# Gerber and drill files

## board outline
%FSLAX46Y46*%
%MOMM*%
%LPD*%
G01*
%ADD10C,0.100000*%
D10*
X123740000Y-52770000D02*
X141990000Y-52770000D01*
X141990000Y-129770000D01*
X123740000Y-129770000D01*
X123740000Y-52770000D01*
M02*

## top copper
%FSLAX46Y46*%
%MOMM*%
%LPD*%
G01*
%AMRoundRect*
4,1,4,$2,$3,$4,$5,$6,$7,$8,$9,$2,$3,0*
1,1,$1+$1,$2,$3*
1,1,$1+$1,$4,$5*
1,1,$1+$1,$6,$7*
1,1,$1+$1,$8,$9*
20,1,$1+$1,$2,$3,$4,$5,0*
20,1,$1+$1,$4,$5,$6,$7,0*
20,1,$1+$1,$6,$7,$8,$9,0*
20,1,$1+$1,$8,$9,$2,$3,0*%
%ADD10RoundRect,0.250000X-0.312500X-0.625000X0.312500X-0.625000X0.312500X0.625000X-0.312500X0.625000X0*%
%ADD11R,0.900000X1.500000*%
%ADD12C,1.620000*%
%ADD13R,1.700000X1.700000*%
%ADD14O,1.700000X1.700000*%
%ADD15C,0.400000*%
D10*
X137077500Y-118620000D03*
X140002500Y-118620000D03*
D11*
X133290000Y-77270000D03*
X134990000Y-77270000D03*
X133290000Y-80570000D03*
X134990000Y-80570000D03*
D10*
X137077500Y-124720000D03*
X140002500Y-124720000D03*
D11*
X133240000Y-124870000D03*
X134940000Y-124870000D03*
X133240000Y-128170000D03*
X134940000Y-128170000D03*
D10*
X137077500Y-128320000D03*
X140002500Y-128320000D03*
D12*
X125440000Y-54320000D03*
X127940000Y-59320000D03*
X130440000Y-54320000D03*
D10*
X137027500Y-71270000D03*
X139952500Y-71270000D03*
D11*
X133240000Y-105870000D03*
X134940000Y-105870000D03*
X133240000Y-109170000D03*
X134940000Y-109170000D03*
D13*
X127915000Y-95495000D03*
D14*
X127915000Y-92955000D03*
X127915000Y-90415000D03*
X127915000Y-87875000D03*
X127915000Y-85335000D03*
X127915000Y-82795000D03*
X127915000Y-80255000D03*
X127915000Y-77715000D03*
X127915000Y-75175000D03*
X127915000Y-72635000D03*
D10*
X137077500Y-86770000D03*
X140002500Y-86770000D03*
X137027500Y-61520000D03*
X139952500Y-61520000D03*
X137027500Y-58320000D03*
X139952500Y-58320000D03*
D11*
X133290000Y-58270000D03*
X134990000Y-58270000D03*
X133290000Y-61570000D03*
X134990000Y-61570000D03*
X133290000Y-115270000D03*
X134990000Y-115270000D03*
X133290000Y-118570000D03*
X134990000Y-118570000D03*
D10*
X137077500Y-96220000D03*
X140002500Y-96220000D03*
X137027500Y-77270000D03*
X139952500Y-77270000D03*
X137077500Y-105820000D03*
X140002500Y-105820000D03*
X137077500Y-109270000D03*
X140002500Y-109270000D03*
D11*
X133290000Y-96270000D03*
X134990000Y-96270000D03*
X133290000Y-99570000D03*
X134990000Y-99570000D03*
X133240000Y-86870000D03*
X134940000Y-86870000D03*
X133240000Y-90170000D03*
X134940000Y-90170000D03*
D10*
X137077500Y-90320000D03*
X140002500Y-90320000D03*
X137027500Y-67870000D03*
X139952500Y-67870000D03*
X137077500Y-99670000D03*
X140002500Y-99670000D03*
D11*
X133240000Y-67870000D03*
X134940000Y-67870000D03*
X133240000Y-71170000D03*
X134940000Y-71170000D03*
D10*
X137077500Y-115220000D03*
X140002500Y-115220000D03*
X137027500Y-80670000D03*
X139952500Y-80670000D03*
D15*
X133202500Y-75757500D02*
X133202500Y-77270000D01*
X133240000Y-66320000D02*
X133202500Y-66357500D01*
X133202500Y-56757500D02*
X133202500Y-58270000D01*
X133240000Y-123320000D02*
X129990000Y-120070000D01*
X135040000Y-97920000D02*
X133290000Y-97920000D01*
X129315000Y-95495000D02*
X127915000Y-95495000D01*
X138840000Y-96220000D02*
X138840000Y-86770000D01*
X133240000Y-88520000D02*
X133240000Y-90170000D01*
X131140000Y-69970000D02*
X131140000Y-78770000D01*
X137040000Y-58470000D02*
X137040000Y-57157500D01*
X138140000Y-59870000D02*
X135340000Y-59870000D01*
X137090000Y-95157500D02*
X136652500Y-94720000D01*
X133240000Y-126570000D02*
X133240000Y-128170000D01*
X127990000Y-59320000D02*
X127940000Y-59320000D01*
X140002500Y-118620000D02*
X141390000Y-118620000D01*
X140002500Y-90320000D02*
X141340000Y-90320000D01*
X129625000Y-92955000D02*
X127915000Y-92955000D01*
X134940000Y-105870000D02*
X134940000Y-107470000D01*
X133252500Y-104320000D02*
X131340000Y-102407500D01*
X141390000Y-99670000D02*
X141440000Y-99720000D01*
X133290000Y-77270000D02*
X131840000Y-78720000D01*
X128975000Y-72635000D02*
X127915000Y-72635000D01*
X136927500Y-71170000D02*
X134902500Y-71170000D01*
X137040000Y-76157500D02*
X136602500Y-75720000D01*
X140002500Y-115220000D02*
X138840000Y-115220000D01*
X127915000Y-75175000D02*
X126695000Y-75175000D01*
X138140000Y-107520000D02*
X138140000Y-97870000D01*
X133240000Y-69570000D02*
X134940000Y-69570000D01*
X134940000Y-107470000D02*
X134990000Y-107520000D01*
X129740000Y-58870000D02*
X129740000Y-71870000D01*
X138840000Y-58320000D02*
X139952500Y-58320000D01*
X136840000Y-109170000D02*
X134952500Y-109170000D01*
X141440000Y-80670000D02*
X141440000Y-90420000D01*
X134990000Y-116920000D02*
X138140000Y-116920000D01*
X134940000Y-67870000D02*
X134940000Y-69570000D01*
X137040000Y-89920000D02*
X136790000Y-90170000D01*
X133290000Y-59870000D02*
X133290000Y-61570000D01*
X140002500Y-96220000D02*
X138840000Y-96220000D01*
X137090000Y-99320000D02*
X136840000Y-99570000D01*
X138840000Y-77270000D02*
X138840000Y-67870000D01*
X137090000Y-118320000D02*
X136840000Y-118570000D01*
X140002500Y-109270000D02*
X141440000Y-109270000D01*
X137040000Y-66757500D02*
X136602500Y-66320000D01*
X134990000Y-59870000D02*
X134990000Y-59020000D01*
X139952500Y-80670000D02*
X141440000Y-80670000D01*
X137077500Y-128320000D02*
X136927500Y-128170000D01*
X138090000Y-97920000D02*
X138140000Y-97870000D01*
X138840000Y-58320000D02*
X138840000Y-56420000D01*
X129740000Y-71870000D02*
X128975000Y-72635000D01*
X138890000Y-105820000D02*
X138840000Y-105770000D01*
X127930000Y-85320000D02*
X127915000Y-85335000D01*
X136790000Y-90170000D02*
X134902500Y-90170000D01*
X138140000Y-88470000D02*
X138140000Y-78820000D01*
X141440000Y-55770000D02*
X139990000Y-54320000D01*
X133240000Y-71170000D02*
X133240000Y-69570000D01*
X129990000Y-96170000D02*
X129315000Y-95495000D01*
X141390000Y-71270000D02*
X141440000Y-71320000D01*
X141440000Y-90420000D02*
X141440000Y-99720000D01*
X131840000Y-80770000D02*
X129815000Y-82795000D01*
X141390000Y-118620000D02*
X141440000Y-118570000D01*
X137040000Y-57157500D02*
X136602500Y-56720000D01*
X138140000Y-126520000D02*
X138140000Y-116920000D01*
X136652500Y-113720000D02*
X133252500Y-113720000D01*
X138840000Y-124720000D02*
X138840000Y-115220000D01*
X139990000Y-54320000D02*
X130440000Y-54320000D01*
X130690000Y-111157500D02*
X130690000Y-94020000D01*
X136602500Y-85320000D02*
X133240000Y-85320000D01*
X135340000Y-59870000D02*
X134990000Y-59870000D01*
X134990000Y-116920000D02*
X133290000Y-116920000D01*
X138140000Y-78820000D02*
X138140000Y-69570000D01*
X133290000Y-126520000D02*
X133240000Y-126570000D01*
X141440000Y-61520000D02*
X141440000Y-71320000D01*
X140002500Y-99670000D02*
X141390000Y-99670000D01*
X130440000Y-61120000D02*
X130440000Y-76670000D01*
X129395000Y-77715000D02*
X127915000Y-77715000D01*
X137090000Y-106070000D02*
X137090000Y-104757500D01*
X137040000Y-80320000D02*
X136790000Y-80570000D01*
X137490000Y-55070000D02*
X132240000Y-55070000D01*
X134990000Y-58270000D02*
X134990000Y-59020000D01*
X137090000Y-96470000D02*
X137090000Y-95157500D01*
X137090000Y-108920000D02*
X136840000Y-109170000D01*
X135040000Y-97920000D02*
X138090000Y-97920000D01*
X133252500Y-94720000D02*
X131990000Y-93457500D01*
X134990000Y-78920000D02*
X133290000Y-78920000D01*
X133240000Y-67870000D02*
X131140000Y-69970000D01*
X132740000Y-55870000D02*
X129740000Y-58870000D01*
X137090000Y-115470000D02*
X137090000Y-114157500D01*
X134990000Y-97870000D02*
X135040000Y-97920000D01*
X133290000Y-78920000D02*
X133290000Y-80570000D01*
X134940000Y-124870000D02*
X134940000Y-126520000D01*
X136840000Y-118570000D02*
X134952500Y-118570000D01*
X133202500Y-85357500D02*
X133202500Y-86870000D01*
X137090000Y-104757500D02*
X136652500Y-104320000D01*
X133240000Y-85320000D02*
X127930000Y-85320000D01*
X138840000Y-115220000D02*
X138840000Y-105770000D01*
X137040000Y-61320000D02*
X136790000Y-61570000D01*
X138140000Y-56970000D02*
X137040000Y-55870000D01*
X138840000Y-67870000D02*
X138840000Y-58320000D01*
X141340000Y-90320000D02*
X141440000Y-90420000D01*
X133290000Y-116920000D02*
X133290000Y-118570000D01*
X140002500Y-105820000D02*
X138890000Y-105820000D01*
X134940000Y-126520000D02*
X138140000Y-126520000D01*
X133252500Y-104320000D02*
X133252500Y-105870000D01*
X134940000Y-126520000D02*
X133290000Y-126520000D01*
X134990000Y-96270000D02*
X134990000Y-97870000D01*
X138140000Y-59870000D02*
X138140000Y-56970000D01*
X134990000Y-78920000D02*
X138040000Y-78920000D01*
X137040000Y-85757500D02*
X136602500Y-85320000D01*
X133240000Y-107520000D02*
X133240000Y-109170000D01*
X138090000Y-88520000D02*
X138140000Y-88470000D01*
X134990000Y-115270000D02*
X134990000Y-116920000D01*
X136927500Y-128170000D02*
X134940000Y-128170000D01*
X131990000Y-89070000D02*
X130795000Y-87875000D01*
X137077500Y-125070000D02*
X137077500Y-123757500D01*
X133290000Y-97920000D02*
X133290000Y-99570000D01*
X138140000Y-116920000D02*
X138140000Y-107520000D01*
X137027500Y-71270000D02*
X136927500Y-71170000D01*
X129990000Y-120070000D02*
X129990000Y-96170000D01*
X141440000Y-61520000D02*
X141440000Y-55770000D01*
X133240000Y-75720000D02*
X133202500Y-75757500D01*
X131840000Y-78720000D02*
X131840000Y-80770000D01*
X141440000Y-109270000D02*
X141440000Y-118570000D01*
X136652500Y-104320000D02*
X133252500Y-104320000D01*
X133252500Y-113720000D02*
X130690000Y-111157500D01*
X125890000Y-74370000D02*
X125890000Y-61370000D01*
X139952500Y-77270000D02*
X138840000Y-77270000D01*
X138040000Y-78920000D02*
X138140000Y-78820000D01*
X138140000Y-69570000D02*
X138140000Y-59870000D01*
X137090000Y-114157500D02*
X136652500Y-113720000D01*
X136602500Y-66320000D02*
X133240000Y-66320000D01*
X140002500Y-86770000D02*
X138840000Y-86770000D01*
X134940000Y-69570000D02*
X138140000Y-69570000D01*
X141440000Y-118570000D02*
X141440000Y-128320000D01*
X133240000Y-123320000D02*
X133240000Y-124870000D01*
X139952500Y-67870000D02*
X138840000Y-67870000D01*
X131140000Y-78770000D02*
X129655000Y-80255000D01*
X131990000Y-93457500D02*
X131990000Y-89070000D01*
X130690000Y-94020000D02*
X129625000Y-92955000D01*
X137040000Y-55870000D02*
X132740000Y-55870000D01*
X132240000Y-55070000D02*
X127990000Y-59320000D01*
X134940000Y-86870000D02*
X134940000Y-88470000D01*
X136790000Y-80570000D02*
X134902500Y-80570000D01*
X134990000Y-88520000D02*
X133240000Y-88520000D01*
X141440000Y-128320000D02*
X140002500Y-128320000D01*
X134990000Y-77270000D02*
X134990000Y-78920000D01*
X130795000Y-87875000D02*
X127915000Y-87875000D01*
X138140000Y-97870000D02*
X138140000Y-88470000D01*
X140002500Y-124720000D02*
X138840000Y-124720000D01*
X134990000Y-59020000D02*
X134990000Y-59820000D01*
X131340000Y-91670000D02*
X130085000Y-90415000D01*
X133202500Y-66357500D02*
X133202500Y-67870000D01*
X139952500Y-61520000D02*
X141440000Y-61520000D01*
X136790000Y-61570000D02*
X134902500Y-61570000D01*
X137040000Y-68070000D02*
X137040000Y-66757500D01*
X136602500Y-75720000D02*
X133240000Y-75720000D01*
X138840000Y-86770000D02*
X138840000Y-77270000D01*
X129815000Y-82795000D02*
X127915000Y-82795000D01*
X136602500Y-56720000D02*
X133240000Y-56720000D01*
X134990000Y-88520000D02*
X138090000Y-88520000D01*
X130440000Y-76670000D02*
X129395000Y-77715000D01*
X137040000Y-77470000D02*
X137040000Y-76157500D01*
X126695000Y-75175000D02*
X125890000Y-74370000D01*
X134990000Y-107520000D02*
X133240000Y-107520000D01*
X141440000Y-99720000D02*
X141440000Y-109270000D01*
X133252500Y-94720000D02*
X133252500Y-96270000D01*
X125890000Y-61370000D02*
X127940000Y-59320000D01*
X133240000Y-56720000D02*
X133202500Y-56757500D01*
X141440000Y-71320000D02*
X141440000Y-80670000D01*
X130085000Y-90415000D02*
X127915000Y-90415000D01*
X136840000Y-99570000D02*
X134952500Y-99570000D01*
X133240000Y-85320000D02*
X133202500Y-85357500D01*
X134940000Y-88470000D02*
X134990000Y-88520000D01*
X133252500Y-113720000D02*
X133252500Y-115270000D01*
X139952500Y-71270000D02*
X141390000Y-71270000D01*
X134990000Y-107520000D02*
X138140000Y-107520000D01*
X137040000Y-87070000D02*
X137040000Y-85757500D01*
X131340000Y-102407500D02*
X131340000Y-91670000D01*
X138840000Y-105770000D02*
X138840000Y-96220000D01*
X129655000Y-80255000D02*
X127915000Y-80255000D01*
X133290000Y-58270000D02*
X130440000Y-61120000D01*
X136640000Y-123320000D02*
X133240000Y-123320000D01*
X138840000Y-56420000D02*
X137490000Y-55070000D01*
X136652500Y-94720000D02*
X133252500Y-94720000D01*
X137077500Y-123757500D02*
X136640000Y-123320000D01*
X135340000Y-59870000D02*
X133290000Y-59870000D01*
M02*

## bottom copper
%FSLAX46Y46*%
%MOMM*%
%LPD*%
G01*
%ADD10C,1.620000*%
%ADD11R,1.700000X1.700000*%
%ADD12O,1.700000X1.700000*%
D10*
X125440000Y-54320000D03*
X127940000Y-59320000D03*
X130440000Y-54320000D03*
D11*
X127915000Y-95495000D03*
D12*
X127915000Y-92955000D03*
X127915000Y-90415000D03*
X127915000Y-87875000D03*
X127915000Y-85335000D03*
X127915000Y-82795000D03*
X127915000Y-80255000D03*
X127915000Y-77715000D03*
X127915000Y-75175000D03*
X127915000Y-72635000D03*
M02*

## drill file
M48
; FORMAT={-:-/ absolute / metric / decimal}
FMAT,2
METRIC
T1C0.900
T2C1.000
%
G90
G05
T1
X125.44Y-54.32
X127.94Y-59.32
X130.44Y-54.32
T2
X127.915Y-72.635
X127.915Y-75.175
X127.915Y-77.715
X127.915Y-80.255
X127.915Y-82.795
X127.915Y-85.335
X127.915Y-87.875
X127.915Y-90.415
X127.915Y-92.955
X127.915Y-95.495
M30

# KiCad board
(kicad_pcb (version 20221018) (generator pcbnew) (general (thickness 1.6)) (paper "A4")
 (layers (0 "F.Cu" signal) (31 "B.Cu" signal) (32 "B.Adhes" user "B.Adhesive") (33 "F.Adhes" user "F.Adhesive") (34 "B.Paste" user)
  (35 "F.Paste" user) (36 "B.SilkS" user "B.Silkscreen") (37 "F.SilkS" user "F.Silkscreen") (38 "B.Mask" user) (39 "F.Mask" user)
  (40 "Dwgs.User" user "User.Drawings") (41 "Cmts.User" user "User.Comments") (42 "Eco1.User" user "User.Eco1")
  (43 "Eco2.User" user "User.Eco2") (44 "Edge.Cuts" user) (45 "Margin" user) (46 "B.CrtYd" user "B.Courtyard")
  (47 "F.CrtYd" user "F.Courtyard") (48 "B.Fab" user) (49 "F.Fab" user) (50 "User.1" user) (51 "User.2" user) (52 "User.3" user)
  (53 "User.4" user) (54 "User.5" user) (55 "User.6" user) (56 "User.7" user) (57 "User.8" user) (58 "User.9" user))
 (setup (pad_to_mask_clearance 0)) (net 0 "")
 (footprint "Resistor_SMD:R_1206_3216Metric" (layer "F.Cu") (at 138.54 118.62)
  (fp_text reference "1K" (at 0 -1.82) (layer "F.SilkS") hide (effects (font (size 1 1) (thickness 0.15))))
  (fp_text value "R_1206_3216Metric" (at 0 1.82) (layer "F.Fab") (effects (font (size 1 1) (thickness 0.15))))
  (pad "1" smd roundrect (at -1.4625 0) (size 1.125 1.75) (layers "F.Cu" "F.Paste" "F.Mask") (roundrect_rratio 0.222222))
  (pad "2" smd roundrect (at 1.4625 0) (size 1.125 1.75) (layers "F.Cu" "F.Paste" "F.Mask") (roundrect_rratio 0.222222)))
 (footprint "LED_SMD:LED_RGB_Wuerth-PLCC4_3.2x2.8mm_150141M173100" (layer "F.Cu") (at 134.14 78.92 90)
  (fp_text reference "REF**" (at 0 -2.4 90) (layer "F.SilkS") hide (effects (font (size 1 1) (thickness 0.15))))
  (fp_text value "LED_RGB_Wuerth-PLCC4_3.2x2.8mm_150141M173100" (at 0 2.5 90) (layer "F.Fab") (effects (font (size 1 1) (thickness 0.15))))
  (pad "1" smd rect (at 1.65 -0.85 90) (size 1.5 0.9) (layers "F.Cu" "F.Paste" "F.Mask"))
  (pad "2" smd rect (at 1.65 0.85 90) (size 1.5 0.9) (layers "F.Cu" "F.Paste" "F.Mask"))
  (pad "3" smd rect (at -1.65 -0.85 90) (size 1.5 0.9) (layers "F.Cu" "F.Paste" "F.Mask"))
  (pad "4" smd rect (at -1.65 0.85 90) (size 1.5 0.9) (layers "F.Cu" "F.Paste" "F.Mask")))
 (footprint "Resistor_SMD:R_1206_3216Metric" (layer "F.Cu") (at 138.54 124.72)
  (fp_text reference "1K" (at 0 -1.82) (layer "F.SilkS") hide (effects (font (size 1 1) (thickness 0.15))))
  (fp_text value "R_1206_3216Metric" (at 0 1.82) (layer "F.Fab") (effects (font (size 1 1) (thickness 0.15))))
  (pad "1" smd roundrect (at -1.4625 0) (size 1.125 1.75) (layers "F.Cu" "F.Paste" "F.Mask") (roundrect_rratio 0.222222))
  (pad "2" smd roundrect (at 1.4625 0) (size 1.125 1.75) (layers "F.Cu" "F.Paste" "F.Mask") (roundrect_rratio 0.222222)))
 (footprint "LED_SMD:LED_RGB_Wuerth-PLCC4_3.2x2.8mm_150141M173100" (layer "F.Cu") (at 134.09 126.52 90)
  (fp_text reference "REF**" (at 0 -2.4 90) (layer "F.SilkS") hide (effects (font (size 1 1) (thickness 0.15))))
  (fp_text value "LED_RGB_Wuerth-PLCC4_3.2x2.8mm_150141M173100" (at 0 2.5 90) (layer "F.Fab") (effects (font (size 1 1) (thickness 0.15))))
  (pad "1" smd rect (at 1.65 -0.85 90) (size 1.5 0.9) (layers "F.Cu" "F.Paste" "F.Mask"))
  (pad "2" smd rect (at 1.65 0.85 90) (size 1.5 0.9) (layers "F.Cu" "F.Paste" "F.Mask"))
  (pad "3" smd rect (at -1.65 -0.85 90) (size 1.5 0.9) (layers "F.Cu" "F.Paste" "F.Mask"))
  (pad "4" smd rect (at -1.65 0.85 90) (size 1.5 0.9) (layers "F.Cu" "F.Paste" "F.Mask")))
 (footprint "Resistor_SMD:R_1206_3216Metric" (layer "F.Cu") (at 138.54 128.32)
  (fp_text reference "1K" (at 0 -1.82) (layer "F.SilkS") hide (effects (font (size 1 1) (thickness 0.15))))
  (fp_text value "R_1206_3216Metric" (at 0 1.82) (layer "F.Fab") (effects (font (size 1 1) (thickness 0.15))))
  (pad "1" smd roundrect (at -1.4625 0) (size 1.125 1.75) (layers "F.Cu" "F.Paste" "F.Mask") (roundrect_rratio 0.222222))
  (pad "2" smd roundrect (at 1.4625 0) (size 1.125 1.75) (layers "F.Cu" "F.Paste" "F.Mask") (roundrect_rratio 0.222222)))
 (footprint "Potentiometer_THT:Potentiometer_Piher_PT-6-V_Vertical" (layer "F.Cu") (at 125.44 54.32 -90)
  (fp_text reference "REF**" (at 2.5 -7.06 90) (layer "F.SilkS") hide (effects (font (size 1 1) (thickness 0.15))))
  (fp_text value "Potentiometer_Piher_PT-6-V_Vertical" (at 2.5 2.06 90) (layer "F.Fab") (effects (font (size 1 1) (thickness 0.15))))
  (pad "1" thru_hole circle (at 0 0 270) (size 1.62 1.62) (drill 0.9) (layers "*.Cu" "*.Mask"))
  (pad "2" thru_hole circle (at 5 -2.5 270) (size 1.62 1.62) (drill 0.9) (layers "*.Cu" "*.Mask"))
  (pad "3" thru_hole circle (at 0 -5 270) (size 1.62 1.62) (drill 0.9) (layers "*.Cu" "*.Mask")))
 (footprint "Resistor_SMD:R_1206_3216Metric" (layer "F.Cu") (at 138.49 71.27)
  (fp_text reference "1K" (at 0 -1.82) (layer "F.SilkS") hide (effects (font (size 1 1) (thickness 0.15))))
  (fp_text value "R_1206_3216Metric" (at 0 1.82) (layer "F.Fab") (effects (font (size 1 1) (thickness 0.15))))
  (pad "1" smd roundrect (at -1.4625 0) (size 1.125 1.75) (layers "F.Cu" "F.Paste" "F.Mask") (roundrect_rratio 0.222222))
  (pad "2" smd roundrect (at 1.4625 0) (size 1.125 1.75) (layers "F.Cu" "F.Paste" "F.Mask") (roundrect_rratio 0.222222)))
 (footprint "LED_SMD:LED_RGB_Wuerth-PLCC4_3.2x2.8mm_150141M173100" (layer "F.Cu") (at 134.09 107.52 90)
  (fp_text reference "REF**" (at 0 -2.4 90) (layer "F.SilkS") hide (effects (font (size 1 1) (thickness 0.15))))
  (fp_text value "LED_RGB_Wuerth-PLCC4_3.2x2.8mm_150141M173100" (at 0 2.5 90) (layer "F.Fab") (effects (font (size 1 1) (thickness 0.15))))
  (pad "1" smd rect (at 1.65 -0.85 90) (size 1.5 0.9) (layers "F.Cu" "F.Paste" "F.Mask"))
  (pad "2" smd rect (at 1.65 0.85 90) (size 1.5 0.9) (layers "F.Cu" "F.Paste" "F.Mask"))
  (pad "3" smd rect (at -1.65 -0.85 90) (size 1.5 0.9) (layers "F.Cu" "F.Paste" "F.Mask"))
  (pad "4" smd rect (at -1.65 0.85 90) (size 1.5 0.9) (layers "F.Cu" "F.Paste" "F.Mask")))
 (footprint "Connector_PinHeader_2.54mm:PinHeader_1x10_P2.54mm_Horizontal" (layer "F.Cu") (at 127.915 95.495 180)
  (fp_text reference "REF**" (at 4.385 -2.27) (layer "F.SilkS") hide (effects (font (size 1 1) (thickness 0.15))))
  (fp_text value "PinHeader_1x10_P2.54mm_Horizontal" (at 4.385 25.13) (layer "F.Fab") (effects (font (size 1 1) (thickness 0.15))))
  (pad "1" thru_hole rect (at 0 0 180) (size 1.7 1.7) (drill 1) (layers "*.Cu" "*.Mask"))
  (pad "2" thru_hole oval (at 0 2.54 180) (size 1.7 1.7) (drill 1) (layers "*.Cu" "*.Mask"))
  (pad "3" thru_hole oval (at 0 5.08 180) (size 1.7 1.7) (drill 1) (layers "*.Cu" "*.Mask"))
  (pad "4" thru_hole oval (at 0 7.62 180) (size 1.7 1.7) (drill 1) (layers "*.Cu" "*.Mask"))
  (pad "5" thru_hole oval (at 0 10.16 180) (size 1.7 1.7) (drill 1) (layers "*.Cu" "*.Mask"))
  (pad "6" thru_hole oval (at 0 12.7 180) (size 1.7 1.7) (drill 1) (layers "*.Cu" "*.Mask"))
  (pad "7" thru_hole oval (at 0 15.24 180) (size 1.7 1.7) (drill 1) (layers "*.Cu" "*.Mask"))
  (pad "8" thru_hole oval (at 0 17.78 180) (size 1.7 1.7) (drill 1) (layers "*.Cu" "*.Mask"))
  (pad "9" thru_hole oval (at 0 20.32 180) (size 1.7 1.7) (drill 1) (layers "*.Cu" "*.Mask"))
  (pad "10" thru_hole oval (at 0 22.86 180) (size 1.7 1.7) (drill 1) (layers "*.Cu" "*.Mask")))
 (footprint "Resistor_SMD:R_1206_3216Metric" (layer "F.Cu") (at 138.54 86.77)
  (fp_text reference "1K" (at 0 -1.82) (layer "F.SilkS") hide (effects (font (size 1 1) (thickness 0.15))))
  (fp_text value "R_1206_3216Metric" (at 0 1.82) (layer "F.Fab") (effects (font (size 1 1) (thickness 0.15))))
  (pad "1" smd roundrect (at -1.4625 0) (size 1.125 1.75) (layers "F.Cu" "F.Paste" "F.Mask") (roundrect_rratio 0.222222))
  (pad "2" smd roundrect (at 1.4625 0) (size 1.125 1.75) (layers "F.Cu" "F.Paste" "F.Mask") (roundrect_rratio 0.222222)))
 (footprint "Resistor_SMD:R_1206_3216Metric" (layer "F.Cu") (at 138.49 61.52)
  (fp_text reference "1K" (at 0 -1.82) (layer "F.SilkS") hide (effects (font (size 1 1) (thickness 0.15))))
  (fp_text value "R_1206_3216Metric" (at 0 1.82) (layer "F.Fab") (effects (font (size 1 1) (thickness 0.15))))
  (pad "1" smd roundrect (at -1.4625 0) (size 1.125 1.75) (layers "F.Cu" "F.Paste" "F.Mask") (roundrect_rratio 0.222222))
  (pad "2" smd roundrect (at 1.4625 0) (size 1.125 1.75) (layers "F.Cu" "F.Paste" "F.Mask") (roundrect_rratio 0.222222)))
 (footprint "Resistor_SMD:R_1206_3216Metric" (layer "F.Cu") (at 138.49 58.32)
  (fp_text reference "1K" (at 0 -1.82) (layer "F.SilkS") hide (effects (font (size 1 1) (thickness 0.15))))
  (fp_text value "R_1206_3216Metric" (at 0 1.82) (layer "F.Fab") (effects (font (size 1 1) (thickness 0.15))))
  (pad "1" smd roundrect (at -1.4625 0) (size 1.125 1.75) (layers "F.Cu" "F.Paste" "F.Mask") (roundrect_rratio 0.222222))
  (pad "2" smd roundrect (at 1.4625 0) (size 1.125 1.75) (layers "F.Cu" "F.Paste" "F.Mask") (roundrect_rratio 0.222222)))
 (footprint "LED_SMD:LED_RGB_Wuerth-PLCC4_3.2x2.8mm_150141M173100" (layer "F.Cu") (at 134.14 59.92 90)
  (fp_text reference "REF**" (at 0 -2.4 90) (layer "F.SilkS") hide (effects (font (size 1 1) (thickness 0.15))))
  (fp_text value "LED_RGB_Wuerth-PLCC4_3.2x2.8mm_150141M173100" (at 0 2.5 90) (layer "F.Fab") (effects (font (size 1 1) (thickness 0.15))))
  (pad "1" smd rect (at 1.65 -0.85 90) (size 1.5 0.9) (layers "F.Cu" "F.Paste" "F.Mask"))
  (pad "2" smd rect (at 1.65 0.85 90) (size 1.5 0.9) (layers "F.Cu" "F.Paste" "F.Mask"))
  (pad "3" smd rect (at -1.65 -0.85 90) (size 1.5 0.9) (layers "F.Cu" "F.Paste" "F.Mask"))
  (pad "4" smd rect (at -1.65 0.85 90) (size 1.5 0.9) (layers "F.Cu" "F.Paste" "F.Mask")))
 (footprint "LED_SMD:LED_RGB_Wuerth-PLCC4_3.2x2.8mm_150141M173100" (layer "F.Cu") (at 134.14 116.92 90)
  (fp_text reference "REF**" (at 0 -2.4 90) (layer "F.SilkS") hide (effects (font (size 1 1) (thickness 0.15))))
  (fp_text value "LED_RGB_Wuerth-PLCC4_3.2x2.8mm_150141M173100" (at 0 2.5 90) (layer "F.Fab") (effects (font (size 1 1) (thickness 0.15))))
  (pad "1" smd rect (at 1.65 -0.85 90) (size 1.5 0.9) (layers "F.Cu" "F.Paste" "F.Mask"))
  (pad "2" smd rect (at 1.65 0.85 90) (size 1.5 0.9) (layers "F.Cu" "F.Paste" "F.Mask"))
  (pad "3" smd rect (at -1.65 -0.85 90) (size 1.5 0.9) (layers "F.Cu" "F.Paste" "F.Mask"))
  (pad "4" smd rect (at -1.65 0.85 90) (size 1.5 0.9) (layers "F.Cu" "F.Paste" "F.Mask")))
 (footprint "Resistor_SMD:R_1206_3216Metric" (layer "F.Cu") (at 138.54 96.22)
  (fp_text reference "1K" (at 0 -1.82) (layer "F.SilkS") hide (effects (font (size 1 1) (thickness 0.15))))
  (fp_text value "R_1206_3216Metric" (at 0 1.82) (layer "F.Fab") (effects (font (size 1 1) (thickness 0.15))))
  (pad "1" smd roundrect (at -1.4625 0) (size 1.125 1.75) (layers "F.Cu" "F.Paste" "F.Mask") (roundrect_rratio 0.222222))
  (pad "2" smd roundrect (at 1.4625 0) (size 1.125 1.75) (layers "F.Cu" "F.Paste" "F.Mask") (roundrect_rratio 0.222222)))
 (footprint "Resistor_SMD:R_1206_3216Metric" (layer "F.Cu") (at 138.49 77.27)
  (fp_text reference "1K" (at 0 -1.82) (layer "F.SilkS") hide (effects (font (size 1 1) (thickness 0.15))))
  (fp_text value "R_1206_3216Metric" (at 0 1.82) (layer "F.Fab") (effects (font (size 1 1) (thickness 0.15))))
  (pad "1" smd roundrect (at -1.4625 0) (size 1.125 1.75) (layers "F.Cu" "F.Paste" "F.Mask") (roundrect_rratio 0.222222))
  (pad "2" smd roundrect (at 1.4625 0) (size 1.125 1.75) (layers "F.Cu" "F.Paste" "F.Mask") (roundrect_rratio 0.222222)))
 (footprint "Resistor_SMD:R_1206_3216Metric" (layer "F.Cu") (at 138.54 105.82)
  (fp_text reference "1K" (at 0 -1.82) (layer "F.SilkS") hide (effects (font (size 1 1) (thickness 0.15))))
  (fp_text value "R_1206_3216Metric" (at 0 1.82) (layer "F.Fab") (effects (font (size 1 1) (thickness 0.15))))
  (pad "1" smd roundrect (at -1.4625 0) (size 1.125 1.75) (layers "F.Cu" "F.Paste" "F.Mask") (roundrect_rratio 0.222222))
  (pad "2" smd roundrect (at 1.4625 0) (size 1.125 1.75) (layers "F.Cu" "F.Paste" "F.Mask") (roundrect_rratio 0.222222)))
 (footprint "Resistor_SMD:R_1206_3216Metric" (layer "F.Cu") (at 138.54 109.27)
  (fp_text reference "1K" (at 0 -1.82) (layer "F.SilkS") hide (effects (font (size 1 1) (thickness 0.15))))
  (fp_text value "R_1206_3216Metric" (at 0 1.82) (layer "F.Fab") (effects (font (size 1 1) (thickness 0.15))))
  (pad "1" smd roundrect (at -1.4625 0) (size 1.125 1.75) (layers "F.Cu" "F.Paste" "F.Mask") (roundrect_rratio 0.222222))
  (pad "2" smd roundrect (at 1.4625 0) (size 1.125 1.75) (layers "F.Cu" "F.Paste" "F.Mask") (roundrect_rratio 0.222222)))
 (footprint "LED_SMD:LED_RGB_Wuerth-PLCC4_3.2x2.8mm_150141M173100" (layer "F.Cu") (at 134.14 97.92 90)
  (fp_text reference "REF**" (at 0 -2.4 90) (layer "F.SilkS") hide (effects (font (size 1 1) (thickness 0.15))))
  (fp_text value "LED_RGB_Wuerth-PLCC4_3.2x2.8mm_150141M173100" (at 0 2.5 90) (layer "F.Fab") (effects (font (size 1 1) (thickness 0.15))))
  (pad "1" smd rect (at 1.65 -0.85 90) (size 1.5 0.9) (layers "F.Cu" "F.Paste" "F.Mask"))
  (pad "2" smd rect (at 1.65 0.85 90) (size 1.5 0.9) (layers "F.Cu" "F.Paste" "F.Mask"))
  (pad "3" smd rect (at -1.65 -0.85 90) (size 1.5 0.9) (layers "F.Cu" "F.Paste" "F.Mask"))
  (pad "4" smd rect (at -1.65 0.85 90) (size 1.5 0.9) (layers "F.Cu" "F.Paste" "F.Mask")))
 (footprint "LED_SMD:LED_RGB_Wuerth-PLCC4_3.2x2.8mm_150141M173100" (layer "F.Cu") (at 134.09 88.52 90)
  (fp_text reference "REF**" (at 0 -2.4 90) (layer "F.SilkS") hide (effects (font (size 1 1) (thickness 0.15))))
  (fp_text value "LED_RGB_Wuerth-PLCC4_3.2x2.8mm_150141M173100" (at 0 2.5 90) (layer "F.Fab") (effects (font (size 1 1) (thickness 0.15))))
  (pad "1" smd rect (at 1.65 -0.85 90) (size 1.5 0.9) (layers "F.Cu" "F.Paste" "F.Mask"))
  (pad "2" smd rect (at 1.65 0.85 90) (size 1.5 0.9) (layers "F.Cu" "F.Paste" "F.Mask"))
  (pad "3" smd rect (at -1.65 -0.85 90) (size 1.5 0.9) (layers "F.Cu" "F.Paste" "F.Mask"))
  (pad "4" smd rect (at -1.65 0.85 90) (size 1.5 0.9) (layers "F.Cu" "F.Paste" "F.Mask")))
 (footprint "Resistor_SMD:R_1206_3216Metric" (layer "F.Cu") (at 138.54 90.32)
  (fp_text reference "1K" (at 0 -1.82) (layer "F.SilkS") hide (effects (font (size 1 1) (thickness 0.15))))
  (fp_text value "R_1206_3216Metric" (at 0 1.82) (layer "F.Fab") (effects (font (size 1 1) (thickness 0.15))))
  (pad "1" smd roundrect (at -1.4625 0) (size 1.125 1.75) (layers "F.Cu" "F.Paste" "F.Mask") (roundrect_rratio 0.222222))
  (pad "2" smd roundrect (at 1.4625 0) (size 1.125 1.75) (layers "F.Cu" "F.Paste" "F.Mask") (roundrect_rratio 0.222222)))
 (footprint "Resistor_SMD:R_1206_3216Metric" (layer "F.Cu") (at 138.49 67.87)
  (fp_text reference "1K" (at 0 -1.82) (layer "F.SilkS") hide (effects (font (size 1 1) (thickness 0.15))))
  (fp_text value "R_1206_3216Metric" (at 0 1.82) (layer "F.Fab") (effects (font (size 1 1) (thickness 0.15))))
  (pad "1" smd roundrect (at -1.4625 0) (size 1.125 1.75) (layers "F.Cu" "F.Paste" "F.Mask") (roundrect_rratio 0.222222))
  (pad "2" smd roundrect (at 1.4625 0) (size 1.125 1.75) (layers "F.Cu" "F.Paste" "F.Mask") (roundrect_rratio 0.222222)))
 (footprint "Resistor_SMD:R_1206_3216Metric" (layer "F.Cu") (at 138.54 99.67)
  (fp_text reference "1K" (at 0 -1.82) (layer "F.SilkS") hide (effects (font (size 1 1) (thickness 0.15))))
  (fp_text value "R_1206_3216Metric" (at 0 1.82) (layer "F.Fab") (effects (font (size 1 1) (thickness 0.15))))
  (pad "1" smd roundrect (at -1.4625 0) (size 1.125 1.75) (layers "F.Cu" "F.Paste" "F.Mask") (roundrect_rratio 0.222222))
  (pad "2" smd roundrect (at 1.4625 0) (size 1.125 1.75) (layers "F.Cu" "F.Paste" "F.Mask") (roundrect_rratio 0.222222)))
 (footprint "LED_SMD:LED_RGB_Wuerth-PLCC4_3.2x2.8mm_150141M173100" (layer "F.Cu") (at 134.09 69.52 90)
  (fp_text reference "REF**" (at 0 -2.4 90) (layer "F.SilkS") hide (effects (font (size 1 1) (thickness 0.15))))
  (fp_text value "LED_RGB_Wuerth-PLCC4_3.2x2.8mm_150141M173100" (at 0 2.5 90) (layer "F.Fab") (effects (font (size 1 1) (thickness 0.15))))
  (pad "1" smd rect (at 1.65 -0.85 90) (size 1.5 0.9) (layers "F.Cu" "F.Paste" "F.Mask"))
  (pad "2" smd rect (at 1.65 0.85 90) (size 1.5 0.9) (layers "F.Cu" "F.Paste" "F.Mask"))
  (pad "3" smd rect (at -1.65 -0.85 90) (size 1.5 0.9) (layers "F.Cu" "F.Paste" "F.Mask"))
  (pad "4" smd rect (at -1.65 0.85 90) (size 1.5 0.9) (layers "F.Cu" "F.Paste" "F.Mask")))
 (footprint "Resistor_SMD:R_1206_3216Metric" (layer "F.Cu") (at 138.54 115.22)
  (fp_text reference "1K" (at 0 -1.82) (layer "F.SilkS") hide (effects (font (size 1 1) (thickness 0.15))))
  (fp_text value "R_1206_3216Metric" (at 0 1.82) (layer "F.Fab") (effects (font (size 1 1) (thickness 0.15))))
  (pad "1" smd roundrect (at -1.4625 0) (size 1.125 1.75) (layers "F.Cu" "F.Paste" "F.Mask") (roundrect_rratio 0.222222))
  (pad "2" smd roundrect (at 1.4625 0) (size 1.125 1.75) (layers "F.Cu" "F.Paste" "F.Mask") (roundrect_rratio 0.222222)))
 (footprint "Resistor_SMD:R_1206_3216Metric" (layer "F.Cu") (at 138.49 80.67)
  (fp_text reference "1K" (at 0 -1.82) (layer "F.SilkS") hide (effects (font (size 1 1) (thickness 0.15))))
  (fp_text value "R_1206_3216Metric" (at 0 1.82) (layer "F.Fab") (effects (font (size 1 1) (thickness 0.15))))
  (pad "1" smd roundrect (at -1.4625 0) (size 1.125 1.75) (layers "F.Cu" "F.Paste" "F.Mask") (roundrect_rratio 0.222222))
  (pad "2" smd roundrect (at 1.4625 0) (size 1.125 1.75) (layers "F.Cu" "F.Paste" "F.Mask") (roundrect_rratio 0.222222)))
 (gr_rect (start 123.74 52.77) (end 141.99 129.77) (stroke (width 0.1) (type solid)) (fill none) (layer "Edge.Cuts"))
 (segment (start 133.2025 75.7575) (end 133.2025 77.27) (width 0.4) (layer "F.Cu") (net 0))
 (segment (start 133.24 66.32) (end 133.2025 66.3575) (width 0.4) (layer "F.Cu") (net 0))
 (segment (start 133.2025 56.7575) (end 133.2025 58.27) (width 0.4) (layer "F.Cu") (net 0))
 (segment (start 133.24 123.32) (end 129.99 120.07) (width 0.4) (layer "F.Cu") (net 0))
 (segment (start 135.04 97.92) (end 133.29 97.92) (width 0.4) (layer "F.Cu") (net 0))
 (segment (start 129.315 95.495) (end 127.915 95.495) (width 0.4) (layer "F.Cu") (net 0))
 (segment (start 138.84 96.22) (end 138.84 86.77) (width 0.4) (layer "F.Cu") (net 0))
 (segment (start 133.24 88.52) (end 133.24 90.17) (width 0.4) (layer "F.Cu") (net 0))
 (segment (start 131.14 69.97) (end 131.14 78.77) (width 0.4) (layer "F.Cu") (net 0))
 (segment (start 137.04 58.47) (end 137.04 57.1575) (width 0.4) (layer "F.Cu") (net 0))
 (segment (start 138.14 59.87) (end 135.34 59.87) (width 0.4) (layer "F.Cu") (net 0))
 (segment (start 137.09 95.1575) (end 136.6525 94.72) (width 0.4) (layer "F.Cu") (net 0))
 (segment (start 133.24 126.57) (end 133.24 128.17) (width 0.4) (layer "F.Cu") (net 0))
 (segment (start 127.99 59.32) (end 127.94 59.32) (width 0.4) (layer "F.Cu") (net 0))
 (segment (start 140.0025 118.62) (end 141.39 118.62) (width 0.4) (layer "F.Cu") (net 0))
 (segment (start 140.0025 90.32) (end 141.34 90.32) (width 0.4) (layer "F.Cu") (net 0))
 (segment (start 129.625 92.955) (end 127.915 92.955) (width 0.4) (layer "F.Cu") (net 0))
 (segment (start 134.94 105.87) (end 134.94 107.47) (width 0.4) (layer "F.Cu") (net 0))
 (segment (start 133.2525 104.32) (end 131.34 102.4075) (width 0.4) (layer "F.Cu") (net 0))
 (segment (start 141.39 99.67) (end 141.44 99.72) (width 0.4) (layer "F.Cu") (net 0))
 (segment (start 133.29 77.27) (end 131.84 78.72) (width 0.4) (layer "F.Cu") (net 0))
 (segment (start 128.975 72.635) (end 127.915 72.635) (width 0.4) (layer "F.Cu") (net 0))
 (segment (start 136.9275 71.17) (end 134.9025 71.17) (width 0.4) (layer "F.Cu") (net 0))
 (segment (start 137.04 76.1575) (end 136.6025 75.72) (width 0.4) (layer "F.Cu") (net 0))
 (segment (start 140.0025 115.22) (end 138.84 115.22) (width 0.4) (layer "F.Cu") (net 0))
 (segment (start 127.915 75.175) (end 126.695 75.175) (width 0.4) (layer "F.Cu") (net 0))
 (segment (start 138.14 107.52) (end 138.14 97.87) (width 0.4) (layer "F.Cu") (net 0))
 (segment (start 133.24 69.57) (end 134.94 69.57) (width 0.4) (layer "F.Cu") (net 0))
 (segment (start 134.94 107.47) (end 134.99 107.52) (width 0.4) (layer "F.Cu") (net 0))
 (segment (start 129.74 58.87) (end 129.74 71.87) (width 0.4) (layer "F.Cu") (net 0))
 (segment (start 138.84 58.32) (end 139.9525 58.32) (width 0.4) (layer "F.Cu") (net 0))
 (segment (start 136.84 109.17) (end 134.9525 109.17) (width 0.4) (layer "F.Cu") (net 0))
 (segment (start 141.44 80.67) (end 141.44 90.42) (width 0.4) (layer "F.Cu") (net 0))
 (segment (start 134.99 116.92) (end 138.14 116.92) (width 0.4) (layer "F.Cu") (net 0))
 (segment (start 134.94 67.87) (end 134.94 69.57) (width 0.4) (layer "F.Cu") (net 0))
 (segment (start 137.04 89.92) (end 136.79 90.17) (width 0.4) (layer "F.Cu") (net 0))
 (segment (start 133.29 59.87) (end 133.29 61.57) (width 0.4) (layer "F.Cu") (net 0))
 (segment (start 140.0025 96.22) (end 138.84 96.22) (width 0.4) (layer "F.Cu") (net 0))
 (segment (start 137.09 99.32) (end 136.84 99.57) (width 0.4) (layer "F.Cu") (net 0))
 (segment (start 138.84 77.27) (end 138.84 67.87) (width 0.4) (layer "F.Cu") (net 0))
 (segment (start 137.09 118.32) (end 136.84 118.57) (width 0.4) (layer "F.Cu") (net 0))
 (segment (start 140.0025 109.27) (end 141.44 109.27) (width 0.4) (layer "F.Cu") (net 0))
 (segment (start 137.04 66.7575) (end 136.6025 66.32) (width 0.4) (layer "F.Cu") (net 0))
 (segment (start 134.99 59.87) (end 134.99 59.02) (width 0.4) (layer "F.Cu") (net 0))
 (segment (start 139.9525 80.67) (end 141.44 80.67) (width 0.4) (layer "F.Cu") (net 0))
 (segment (start 137.0775 128.32) (end 136.9275 128.17) (width 0.4) (layer "F.Cu") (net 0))
 (segment (start 138.09 97.92) (end 138.14 97.87) (width 0.4) (layer "F.Cu") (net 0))
 (segment (start 138.84 58.32) (end 138.84 56.42) (width 0.4) (layer "F.Cu") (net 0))
 (segment (start 129.74 71.87) (end 128.975 72.635) (width 0.4) (layer "F.Cu") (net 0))
 (segment (start 138.89 105.82) (end 138.84 105.77) (width 0.4) (layer "F.Cu") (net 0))
 (segment (start 127.93 85.32) (end 127.915 85.335) (width 0.4) (layer "F.Cu") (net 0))
 (segment (start 136.79 90.17) (end 134.9025 90.17) (width 0.4) (layer "F.Cu") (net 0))
 (segment (start 138.14 88.47) (end 138.14 78.82) (width 0.4) (layer "F.Cu") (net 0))
 (segment (start 141.44 55.77) (end 139.99 54.32) (width 0.4) (layer "F.Cu") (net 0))
 (segment (start 133.24 71.17) (end 133.24 69.57) (width 0.4) (layer "F.Cu") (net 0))
 (segment (start 129.99 96.17) (end 129.315 95.495) (width 0.4) (layer "F.Cu") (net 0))
 (segment (start 141.39 71.27) (end 141.44 71.32) (width 0.4) (layer "F.Cu") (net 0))
 (segment (start 141.44 90.42) (end 141.44 99.72) (width 0.4) (layer "F.Cu") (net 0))
 (segment (start 131.84 80.77) (end 129.815 82.795) (width 0.4) (layer "F.Cu") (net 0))
 (segment (start 141.39 118.62) (end 141.44 118.57) (width 0.4) (layer "F.Cu") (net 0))
 (segment (start 137.04 57.1575) (end 136.6025 56.72) (width 0.4) (layer "F.Cu") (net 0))
 (segment (start 138.14 126.52) (end 138.14 116.92) (width 0.4) (layer "F.Cu") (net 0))
 (segment (start 136.6525 113.72) (end 133.2525 113.72) (width 0.4) (layer "F.Cu") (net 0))
 (segment (start 138.84 124.72) (end 138.84 115.22) (width 0.4) (layer "F.Cu") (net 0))
 (segment (start 139.99 54.32) (end 130.44 54.32) (width 0.4) (layer "F.Cu") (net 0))
 (segment (start 130.69 111.1575) (end 130.69 94.02) (width 0.4) (layer "F.Cu") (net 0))
 (segment (start 136.6025 85.32) (end 133.24 85.32) (width 0.4) (layer "F.Cu") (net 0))
 (segment (start 135.34 59.87) (end 134.99 59.87) (width 0.4) (layer "F.Cu") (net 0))
 (segment (start 134.99 116.92) (end 133.29 116.92) (width 0.4) (layer "F.Cu") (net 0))
 (segment (start 138.14 78.82) (end 138.14 69.57) (width 0.4) (layer "F.Cu") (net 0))
 (segment (start 133.29 126.52) (end 133.24 126.57) (width 0.4) (layer "F.Cu") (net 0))
 (segment (start 141.44 61.52) (end 141.44 71.32) (width 0.4) (layer "F.Cu") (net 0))
 (segment (start 140.0025 99.67) (end 141.39 99.67) (width 0.4) (layer "F.Cu") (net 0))
 (segment (start 130.44 61.12) (end 130.44 76.67) (width 0.4) (layer "F.Cu") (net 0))
 (segment (start 129.395 77.715) (end 127.915 77.715) (width 0.4) (layer "F.Cu") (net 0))
 (segment (start 137.09 106.07) (end 137.09 104.7575) (width 0.4) (layer "F.Cu") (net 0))
 (segment (start 137.04 80.32) (end 136.79 80.57) (width 0.4) (layer "F.Cu") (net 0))
 (segment (start 137.49 55.07) (end 132.24 55.07) (width 0.4) (layer "F.Cu") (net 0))
 (segment (start 134.99 58.27) (end 134.99 59.02) (width 0.4) (layer "F.Cu") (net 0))
 (segment (start 137.09 96.47) (end 137.09 95.1575) (width 0.4) (layer "F.Cu") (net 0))
 (segment (start 137.09 108.92) (end 136.84 109.17) (width 0.4) (layer "F.Cu") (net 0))
 (segment (start 135.04 97.92) (end 138.09 97.92) (width 0.4) (layer "F.Cu") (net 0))
 (segment (start 133.2525 94.72) (end 131.99 93.4575) (width 0.4) (layer "F.Cu") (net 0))
 (segment (start 134.99 78.92) (end 133.29 78.92) (width 0.4) (layer "F.Cu") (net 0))
 (segment (start 133.24 67.87) (end 131.14 69.97) (width 0.4) (layer "F.Cu") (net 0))
 (segment (start 132.74 55.87) (end 129.74 58.87) (width 0.4) (layer "F.Cu") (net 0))
 (segment (start 137.09 115.47) (end 137.09 114.1575) (width 0.4) (layer "F.Cu") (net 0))
 (segment (start 134.99 97.87) (end 135.04 97.92) (width 0.4) (layer "F.Cu") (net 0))
 (segment (start 133.29 78.92) (end 133.29 80.57) (width 0.4) (layer "F.Cu") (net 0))
 (segment (start 134.94 124.87) (end 134.94 126.52) (width 0.4) (layer "F.Cu") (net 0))
 (segment (start 136.84 118.57) (end 134.9525 118.57) (width 0.4) (layer "F.Cu") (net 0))
 (segment (start 133.2025 85.3575) (end 133.2025 86.87) (width 0.4) (layer "F.Cu") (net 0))
 (segment (start 137.09 104.7575) (end 136.6525 104.32) (width 0.4) (layer "F.Cu") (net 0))
 (segment (start 133.24 85.32) (end 127.93 85.32) (width 0.4) (layer "F.Cu") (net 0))
 (segment (start 138.84 115.22) (end 138.84 105.77) (width 0.4) (layer "F.Cu") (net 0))
 (segment (start 137.04 61.32) (end 136.79 61.57) (width 0.4) (layer "F.Cu") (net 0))
 (segment (start 138.14 56.97) (end 137.04 55.87) (width 0.4) (layer "F.Cu") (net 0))
 (segment (start 138.84 67.87) (end 138.84 58.32) (width 0.4) (layer "F.Cu") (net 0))
 (segment (start 141.34 90.32) (end 141.44 90.42) (width 0.4) (layer "F.Cu") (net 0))
 (segment (start 133.29 116.92) (end 133.29 118.57) (width 0.4) (layer "F.Cu") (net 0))
 (segment (start 140.0025 105.82) (end 138.89 105.82) (width 0.4) (layer "F.Cu") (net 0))
 (segment (start 134.94 126.52) (end 138.14 126.52) (width 0.4) (layer "F.Cu") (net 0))
 (segment (start 133.2525 104.32) (end 133.2525 105.87) (width 0.4) (layer "F.Cu") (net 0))
 (segment (start 134.94 126.52) (end 133.29 126.52) (width 0.4) (layer "F.Cu") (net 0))
 (segment (start 134.99 96.27) (end 134.99 97.87) (width 0.4) (layer "F.Cu") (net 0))
 (segment (start 138.14 59.87) (end 138.14 56.97) (width 0.4) (layer "F.Cu") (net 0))
 (segment (start 134.99 78.92) (end 138.04 78.92) (width 0.4) (layer "F.Cu") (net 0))
 (segment (start 137.04 85.7575) (end 136.6025 85.32) (width 0.4) (layer "F.Cu") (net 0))
 (segment (start 133.24 107.52) (end 133.24 109.17) (width 0.4) (layer "F.Cu") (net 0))
 (segment (start 138.09 88.52) (end 138.14 88.47) (width 0.4) (layer "F.Cu") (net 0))
 (segment (start 134.99 115.27) (end 134.99 116.92) (width 0.4) (layer "F.Cu") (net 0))
 (segment (start 136.9275 128.17) (end 134.94 128.17) (width 0.4) (layer "F.Cu") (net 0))
 (segment (start 131.99 89.07) (end 130.795 87.875) (width 0.4) (layer "F.Cu") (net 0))
 (segment (start 137.0775 125.07) (end 137.0775 123.7575) (width 0.4) (layer "F.Cu") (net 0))
 (segment (start 133.29 97.92) (end 133.29 99.57) (width 0.4) (layer "F.Cu") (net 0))
 (segment (start 138.14 116.92) (end 138.14 107.52) (width 0.4) (layer "F.Cu") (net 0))
 (segment (start 137.0275 71.27) (end 136.9275 71.17) (width 0.4) (layer "F.Cu") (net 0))
 (segment (start 129.99 120.07) (end 129.99 96.17) (width 0.4) (layer "F.Cu") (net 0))
 (segment (start 141.44 61.52) (end 141.44 55.77) (width 0.4) (layer "F.Cu") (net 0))
 (segment (start 133.24 75.72) (end 133.2025 75.7575) (width 0.4) (layer "F.Cu") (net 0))
 (segment (start 131.84 78.72) (end 131.84 80.77) (width 0.4) (layer "F.Cu") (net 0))
 (segment (start 141.44 109.27) (end 141.44 118.57) (width 0.4) (layer "F.Cu") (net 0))
 (segment (start 136.6525 104.32) (end 133.2525 104.32) (width 0.4) (layer "F.Cu") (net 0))
 (segment (start 133.2525 113.72) (end 130.69 111.1575) (width 0.4) (layer "F.Cu") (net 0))
 (segment (start 125.89 74.37) (end 125.89 61.37) (width 0.4) (layer "F.Cu") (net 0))
 (segment (start 139.9525 77.27) (end 138.84 77.27) (width 0.4) (layer "F.Cu") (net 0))
 (segment (start 138.04 78.92) (end 138.14 78.82) (width 0.4) (layer "F.Cu") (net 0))
 (segment (start 138.14 69.57) (end 138.14 59.87) (width 0.4) (layer "F.Cu") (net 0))
 (segment (start 137.09 114.1575) (end 136.6525 113.72) (width 0.4) (layer "F.Cu") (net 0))
 (segment (start 136.6025 66.32) (end 133.24 66.32) (width 0.4) (layer "F.Cu") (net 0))
 (segment (start 140.0025 86.77) (end 138.84 86.77) (width 0.4) (layer "F.Cu") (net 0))
 (segment (start 134.94 69.57) (end 138.14 69.57) (width 0.4) (layer "F.Cu") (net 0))
 (segment (start 141.44 118.57) (end 141.44 128.32) (width 0.4) (layer "F.Cu") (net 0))
 (segment (start 133.24 123.32) (end 133.24 124.87) (width 0.4) (layer "F.Cu") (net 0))
 (segment (start 139.9525 67.87) (end 138.84 67.87) (width 0.4) (layer "F.Cu") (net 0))
 (segment (start 131.14 78.77) (end 129.655 80.255) (width 0.4) (layer "F.Cu") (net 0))
 (segment (start 131.99 93.4575) (end 131.99 89.07) (width 0.4) (layer "F.Cu") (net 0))
 (segment (start 130.69 94.02) (end 129.625 92.955) (width 0.4) (layer "F.Cu") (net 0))
 (segment (start 137.04 55.87) (end 132.74 55.87) (width 0.4) (layer "F.Cu") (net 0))
 (segment (start 132.24 55.07) (end 127.99 59.32) (width 0.4) (layer "F.Cu") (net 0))
 (segment (start 134.94 86.87) (end 134.94 88.47) (width 0.4) (layer "F.Cu") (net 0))
 (segment (start 136.79 80.57) (end 134.9025 80.57) (width 0.4) (layer "F.Cu") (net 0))
 (segment (start 134.99 88.52) (end 133.24 88.52) (width 0.4) (layer "F.Cu") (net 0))
 (segment (start 141.44 128.32) (end 140.0025 128.32) (width 0.4) (layer "F.Cu") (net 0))
 (segment (start 134.99 77.27) (end 134.99 78.92) (width 0.4) (layer "F.Cu") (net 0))
 (segment (start 130.795 87.875) (end 127.915 87.875) (width 0.4) (layer "F.Cu") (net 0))
 (segment (start 138.14 97.87) (end 138.14 88.47) (width 0.4) (layer "F.Cu") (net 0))
 (segment (start 140.0025 124.72) (end 138.84 124.72) (width 0.4) (layer "F.Cu") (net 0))
 (segment (start 134.99 59.02) (end 134.99 59.82) (width 0.4) (layer "F.Cu") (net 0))
 (segment (start 131.34 91.67) (end 130.085 90.415) (width 0.4) (layer "F.Cu") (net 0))
 (segment (start 133.2025 66.3575) (end 133.2025 67.87) (width 0.4) (layer "F.Cu") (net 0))
 (segment (start 139.9525 61.52) (end 141.44 61.52) (width 0.4) (layer "F.Cu") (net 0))
 (segment (start 136.79 61.57) (end 134.9025 61.57) (width 0.4) (layer "F.Cu") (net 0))
 (segment (start 137.04 68.07) (end 137.04 66.7575) (width 0.4) (layer "F.Cu") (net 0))
 (segment (start 136.6025 75.72) (end 133.24 75.72) (width 0.4) (layer "F.Cu") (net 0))
 (segment (start 138.84 86.77) (end 138.84 77.27) (width 0.4) (layer "F.Cu") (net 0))
 (segment (start 129.815 82.795) (end 127.915 82.795) (width 0.4) (layer "F.Cu") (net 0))
 (segment (start 136.6025 56.72) (end 133.24 56.72) (width 0.4) (layer "F.Cu") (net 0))
 (segment (start 134.99 88.52) (end 138.09 88.52) (width 0.4) (layer "F.Cu") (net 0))
 (segment (start 130.44 76.67) (end 129.395 77.715) (width 0.4) (layer "F.Cu") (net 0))
 (segment (start 137.04 77.47) (end 137.04 76.1575) (width 0.4) (layer "F.Cu") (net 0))
 (segment (start 126.695 75.175) (end 125.89 74.37) (width 0.4) (layer "F.Cu") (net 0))
 (segment (start 134.99 107.52) (end 133.24 107.52) (width 0.4) (layer "F.Cu") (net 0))
 (segment (start 141.44 99.72) (end 141.44 109.27) (width 0.4) (layer "F.Cu") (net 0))
 (segment (start 133.2525 94.72) (end 133.2525 96.27) (width 0.4) (layer "F.Cu") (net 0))
 (segment (start 125.89 61.37) (end 127.94 59.32) (width 0.4) (layer "F.Cu") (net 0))
 (segment (start 133.24 56.72) (end 133.2025 56.7575) (width 0.4) (layer "F.Cu") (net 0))
 (segment (start 141.44 71.32) (end 141.44 80.67) (width 0.4) (layer "F.Cu") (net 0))
 (segment (start 130.085 90.415) (end 127.915 90.415) (width 0.4) (layer "F.Cu") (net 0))
 (segment (start 136.84 99.57) (end 134.9525 99.57) (width 0.4) (layer "F.Cu") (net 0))
 (segment (start 133.24 85.32) (end 133.2025 85.3575) (width 0.4) (layer "F.Cu") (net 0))
 (segment (start 134.94 88.47) (end 134.99 88.52) (width 0.4) (layer "F.Cu") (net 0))
 (segment (start 133.2525 113.72) (end 133.2525 115.27) (width 0.4) (layer "F.Cu") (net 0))
 (segment (start 139.9525 71.27) (end 141.39 71.27) (width 0.4) (layer "F.Cu") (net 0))
 (segment (start 134.99 107.52) (end 138.14 107.52) (width 0.4) (layer "F.Cu") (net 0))
 (segment (start 137.04 87.07) (end 137.04 85.7575) (width 0.4) (layer "F.Cu") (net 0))
 (segment (start 131.34 102.4075) (end 131.34 91.67) (width 0.4) (layer "F.Cu") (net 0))
 (segment (start 138.84 105.77) (end 138.84 96.22) (width 0.4) (layer "F.Cu") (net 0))
 (segment (start 129.655 80.255) (end 127.915 80.255) (width 0.4) (layer "F.Cu") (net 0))
 (segment (start 133.29 58.27) (end 130.44 61.12) (width 0.4) (layer "F.Cu") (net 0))
 (segment (start 136.64 123.32) (end 133.24 123.32) (width 0.4) (layer "F.Cu") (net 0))
 (segment (start 138.84 56.42) (end 137.49 55.07) (width 0.4) (layer "F.Cu") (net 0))
 (segment (start 136.6525 94.72) (end 133.2525 94.72) (width 0.4) (layer "F.Cu") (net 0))
 (segment (start 137.0775 123.7575) (end 136.64 123.32) (width 0.4) (layer "F.Cu") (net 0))
 (segment (start 135.34 59.87) (end 133.29 59.87) (width 0.4) (layer "F.Cu") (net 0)))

